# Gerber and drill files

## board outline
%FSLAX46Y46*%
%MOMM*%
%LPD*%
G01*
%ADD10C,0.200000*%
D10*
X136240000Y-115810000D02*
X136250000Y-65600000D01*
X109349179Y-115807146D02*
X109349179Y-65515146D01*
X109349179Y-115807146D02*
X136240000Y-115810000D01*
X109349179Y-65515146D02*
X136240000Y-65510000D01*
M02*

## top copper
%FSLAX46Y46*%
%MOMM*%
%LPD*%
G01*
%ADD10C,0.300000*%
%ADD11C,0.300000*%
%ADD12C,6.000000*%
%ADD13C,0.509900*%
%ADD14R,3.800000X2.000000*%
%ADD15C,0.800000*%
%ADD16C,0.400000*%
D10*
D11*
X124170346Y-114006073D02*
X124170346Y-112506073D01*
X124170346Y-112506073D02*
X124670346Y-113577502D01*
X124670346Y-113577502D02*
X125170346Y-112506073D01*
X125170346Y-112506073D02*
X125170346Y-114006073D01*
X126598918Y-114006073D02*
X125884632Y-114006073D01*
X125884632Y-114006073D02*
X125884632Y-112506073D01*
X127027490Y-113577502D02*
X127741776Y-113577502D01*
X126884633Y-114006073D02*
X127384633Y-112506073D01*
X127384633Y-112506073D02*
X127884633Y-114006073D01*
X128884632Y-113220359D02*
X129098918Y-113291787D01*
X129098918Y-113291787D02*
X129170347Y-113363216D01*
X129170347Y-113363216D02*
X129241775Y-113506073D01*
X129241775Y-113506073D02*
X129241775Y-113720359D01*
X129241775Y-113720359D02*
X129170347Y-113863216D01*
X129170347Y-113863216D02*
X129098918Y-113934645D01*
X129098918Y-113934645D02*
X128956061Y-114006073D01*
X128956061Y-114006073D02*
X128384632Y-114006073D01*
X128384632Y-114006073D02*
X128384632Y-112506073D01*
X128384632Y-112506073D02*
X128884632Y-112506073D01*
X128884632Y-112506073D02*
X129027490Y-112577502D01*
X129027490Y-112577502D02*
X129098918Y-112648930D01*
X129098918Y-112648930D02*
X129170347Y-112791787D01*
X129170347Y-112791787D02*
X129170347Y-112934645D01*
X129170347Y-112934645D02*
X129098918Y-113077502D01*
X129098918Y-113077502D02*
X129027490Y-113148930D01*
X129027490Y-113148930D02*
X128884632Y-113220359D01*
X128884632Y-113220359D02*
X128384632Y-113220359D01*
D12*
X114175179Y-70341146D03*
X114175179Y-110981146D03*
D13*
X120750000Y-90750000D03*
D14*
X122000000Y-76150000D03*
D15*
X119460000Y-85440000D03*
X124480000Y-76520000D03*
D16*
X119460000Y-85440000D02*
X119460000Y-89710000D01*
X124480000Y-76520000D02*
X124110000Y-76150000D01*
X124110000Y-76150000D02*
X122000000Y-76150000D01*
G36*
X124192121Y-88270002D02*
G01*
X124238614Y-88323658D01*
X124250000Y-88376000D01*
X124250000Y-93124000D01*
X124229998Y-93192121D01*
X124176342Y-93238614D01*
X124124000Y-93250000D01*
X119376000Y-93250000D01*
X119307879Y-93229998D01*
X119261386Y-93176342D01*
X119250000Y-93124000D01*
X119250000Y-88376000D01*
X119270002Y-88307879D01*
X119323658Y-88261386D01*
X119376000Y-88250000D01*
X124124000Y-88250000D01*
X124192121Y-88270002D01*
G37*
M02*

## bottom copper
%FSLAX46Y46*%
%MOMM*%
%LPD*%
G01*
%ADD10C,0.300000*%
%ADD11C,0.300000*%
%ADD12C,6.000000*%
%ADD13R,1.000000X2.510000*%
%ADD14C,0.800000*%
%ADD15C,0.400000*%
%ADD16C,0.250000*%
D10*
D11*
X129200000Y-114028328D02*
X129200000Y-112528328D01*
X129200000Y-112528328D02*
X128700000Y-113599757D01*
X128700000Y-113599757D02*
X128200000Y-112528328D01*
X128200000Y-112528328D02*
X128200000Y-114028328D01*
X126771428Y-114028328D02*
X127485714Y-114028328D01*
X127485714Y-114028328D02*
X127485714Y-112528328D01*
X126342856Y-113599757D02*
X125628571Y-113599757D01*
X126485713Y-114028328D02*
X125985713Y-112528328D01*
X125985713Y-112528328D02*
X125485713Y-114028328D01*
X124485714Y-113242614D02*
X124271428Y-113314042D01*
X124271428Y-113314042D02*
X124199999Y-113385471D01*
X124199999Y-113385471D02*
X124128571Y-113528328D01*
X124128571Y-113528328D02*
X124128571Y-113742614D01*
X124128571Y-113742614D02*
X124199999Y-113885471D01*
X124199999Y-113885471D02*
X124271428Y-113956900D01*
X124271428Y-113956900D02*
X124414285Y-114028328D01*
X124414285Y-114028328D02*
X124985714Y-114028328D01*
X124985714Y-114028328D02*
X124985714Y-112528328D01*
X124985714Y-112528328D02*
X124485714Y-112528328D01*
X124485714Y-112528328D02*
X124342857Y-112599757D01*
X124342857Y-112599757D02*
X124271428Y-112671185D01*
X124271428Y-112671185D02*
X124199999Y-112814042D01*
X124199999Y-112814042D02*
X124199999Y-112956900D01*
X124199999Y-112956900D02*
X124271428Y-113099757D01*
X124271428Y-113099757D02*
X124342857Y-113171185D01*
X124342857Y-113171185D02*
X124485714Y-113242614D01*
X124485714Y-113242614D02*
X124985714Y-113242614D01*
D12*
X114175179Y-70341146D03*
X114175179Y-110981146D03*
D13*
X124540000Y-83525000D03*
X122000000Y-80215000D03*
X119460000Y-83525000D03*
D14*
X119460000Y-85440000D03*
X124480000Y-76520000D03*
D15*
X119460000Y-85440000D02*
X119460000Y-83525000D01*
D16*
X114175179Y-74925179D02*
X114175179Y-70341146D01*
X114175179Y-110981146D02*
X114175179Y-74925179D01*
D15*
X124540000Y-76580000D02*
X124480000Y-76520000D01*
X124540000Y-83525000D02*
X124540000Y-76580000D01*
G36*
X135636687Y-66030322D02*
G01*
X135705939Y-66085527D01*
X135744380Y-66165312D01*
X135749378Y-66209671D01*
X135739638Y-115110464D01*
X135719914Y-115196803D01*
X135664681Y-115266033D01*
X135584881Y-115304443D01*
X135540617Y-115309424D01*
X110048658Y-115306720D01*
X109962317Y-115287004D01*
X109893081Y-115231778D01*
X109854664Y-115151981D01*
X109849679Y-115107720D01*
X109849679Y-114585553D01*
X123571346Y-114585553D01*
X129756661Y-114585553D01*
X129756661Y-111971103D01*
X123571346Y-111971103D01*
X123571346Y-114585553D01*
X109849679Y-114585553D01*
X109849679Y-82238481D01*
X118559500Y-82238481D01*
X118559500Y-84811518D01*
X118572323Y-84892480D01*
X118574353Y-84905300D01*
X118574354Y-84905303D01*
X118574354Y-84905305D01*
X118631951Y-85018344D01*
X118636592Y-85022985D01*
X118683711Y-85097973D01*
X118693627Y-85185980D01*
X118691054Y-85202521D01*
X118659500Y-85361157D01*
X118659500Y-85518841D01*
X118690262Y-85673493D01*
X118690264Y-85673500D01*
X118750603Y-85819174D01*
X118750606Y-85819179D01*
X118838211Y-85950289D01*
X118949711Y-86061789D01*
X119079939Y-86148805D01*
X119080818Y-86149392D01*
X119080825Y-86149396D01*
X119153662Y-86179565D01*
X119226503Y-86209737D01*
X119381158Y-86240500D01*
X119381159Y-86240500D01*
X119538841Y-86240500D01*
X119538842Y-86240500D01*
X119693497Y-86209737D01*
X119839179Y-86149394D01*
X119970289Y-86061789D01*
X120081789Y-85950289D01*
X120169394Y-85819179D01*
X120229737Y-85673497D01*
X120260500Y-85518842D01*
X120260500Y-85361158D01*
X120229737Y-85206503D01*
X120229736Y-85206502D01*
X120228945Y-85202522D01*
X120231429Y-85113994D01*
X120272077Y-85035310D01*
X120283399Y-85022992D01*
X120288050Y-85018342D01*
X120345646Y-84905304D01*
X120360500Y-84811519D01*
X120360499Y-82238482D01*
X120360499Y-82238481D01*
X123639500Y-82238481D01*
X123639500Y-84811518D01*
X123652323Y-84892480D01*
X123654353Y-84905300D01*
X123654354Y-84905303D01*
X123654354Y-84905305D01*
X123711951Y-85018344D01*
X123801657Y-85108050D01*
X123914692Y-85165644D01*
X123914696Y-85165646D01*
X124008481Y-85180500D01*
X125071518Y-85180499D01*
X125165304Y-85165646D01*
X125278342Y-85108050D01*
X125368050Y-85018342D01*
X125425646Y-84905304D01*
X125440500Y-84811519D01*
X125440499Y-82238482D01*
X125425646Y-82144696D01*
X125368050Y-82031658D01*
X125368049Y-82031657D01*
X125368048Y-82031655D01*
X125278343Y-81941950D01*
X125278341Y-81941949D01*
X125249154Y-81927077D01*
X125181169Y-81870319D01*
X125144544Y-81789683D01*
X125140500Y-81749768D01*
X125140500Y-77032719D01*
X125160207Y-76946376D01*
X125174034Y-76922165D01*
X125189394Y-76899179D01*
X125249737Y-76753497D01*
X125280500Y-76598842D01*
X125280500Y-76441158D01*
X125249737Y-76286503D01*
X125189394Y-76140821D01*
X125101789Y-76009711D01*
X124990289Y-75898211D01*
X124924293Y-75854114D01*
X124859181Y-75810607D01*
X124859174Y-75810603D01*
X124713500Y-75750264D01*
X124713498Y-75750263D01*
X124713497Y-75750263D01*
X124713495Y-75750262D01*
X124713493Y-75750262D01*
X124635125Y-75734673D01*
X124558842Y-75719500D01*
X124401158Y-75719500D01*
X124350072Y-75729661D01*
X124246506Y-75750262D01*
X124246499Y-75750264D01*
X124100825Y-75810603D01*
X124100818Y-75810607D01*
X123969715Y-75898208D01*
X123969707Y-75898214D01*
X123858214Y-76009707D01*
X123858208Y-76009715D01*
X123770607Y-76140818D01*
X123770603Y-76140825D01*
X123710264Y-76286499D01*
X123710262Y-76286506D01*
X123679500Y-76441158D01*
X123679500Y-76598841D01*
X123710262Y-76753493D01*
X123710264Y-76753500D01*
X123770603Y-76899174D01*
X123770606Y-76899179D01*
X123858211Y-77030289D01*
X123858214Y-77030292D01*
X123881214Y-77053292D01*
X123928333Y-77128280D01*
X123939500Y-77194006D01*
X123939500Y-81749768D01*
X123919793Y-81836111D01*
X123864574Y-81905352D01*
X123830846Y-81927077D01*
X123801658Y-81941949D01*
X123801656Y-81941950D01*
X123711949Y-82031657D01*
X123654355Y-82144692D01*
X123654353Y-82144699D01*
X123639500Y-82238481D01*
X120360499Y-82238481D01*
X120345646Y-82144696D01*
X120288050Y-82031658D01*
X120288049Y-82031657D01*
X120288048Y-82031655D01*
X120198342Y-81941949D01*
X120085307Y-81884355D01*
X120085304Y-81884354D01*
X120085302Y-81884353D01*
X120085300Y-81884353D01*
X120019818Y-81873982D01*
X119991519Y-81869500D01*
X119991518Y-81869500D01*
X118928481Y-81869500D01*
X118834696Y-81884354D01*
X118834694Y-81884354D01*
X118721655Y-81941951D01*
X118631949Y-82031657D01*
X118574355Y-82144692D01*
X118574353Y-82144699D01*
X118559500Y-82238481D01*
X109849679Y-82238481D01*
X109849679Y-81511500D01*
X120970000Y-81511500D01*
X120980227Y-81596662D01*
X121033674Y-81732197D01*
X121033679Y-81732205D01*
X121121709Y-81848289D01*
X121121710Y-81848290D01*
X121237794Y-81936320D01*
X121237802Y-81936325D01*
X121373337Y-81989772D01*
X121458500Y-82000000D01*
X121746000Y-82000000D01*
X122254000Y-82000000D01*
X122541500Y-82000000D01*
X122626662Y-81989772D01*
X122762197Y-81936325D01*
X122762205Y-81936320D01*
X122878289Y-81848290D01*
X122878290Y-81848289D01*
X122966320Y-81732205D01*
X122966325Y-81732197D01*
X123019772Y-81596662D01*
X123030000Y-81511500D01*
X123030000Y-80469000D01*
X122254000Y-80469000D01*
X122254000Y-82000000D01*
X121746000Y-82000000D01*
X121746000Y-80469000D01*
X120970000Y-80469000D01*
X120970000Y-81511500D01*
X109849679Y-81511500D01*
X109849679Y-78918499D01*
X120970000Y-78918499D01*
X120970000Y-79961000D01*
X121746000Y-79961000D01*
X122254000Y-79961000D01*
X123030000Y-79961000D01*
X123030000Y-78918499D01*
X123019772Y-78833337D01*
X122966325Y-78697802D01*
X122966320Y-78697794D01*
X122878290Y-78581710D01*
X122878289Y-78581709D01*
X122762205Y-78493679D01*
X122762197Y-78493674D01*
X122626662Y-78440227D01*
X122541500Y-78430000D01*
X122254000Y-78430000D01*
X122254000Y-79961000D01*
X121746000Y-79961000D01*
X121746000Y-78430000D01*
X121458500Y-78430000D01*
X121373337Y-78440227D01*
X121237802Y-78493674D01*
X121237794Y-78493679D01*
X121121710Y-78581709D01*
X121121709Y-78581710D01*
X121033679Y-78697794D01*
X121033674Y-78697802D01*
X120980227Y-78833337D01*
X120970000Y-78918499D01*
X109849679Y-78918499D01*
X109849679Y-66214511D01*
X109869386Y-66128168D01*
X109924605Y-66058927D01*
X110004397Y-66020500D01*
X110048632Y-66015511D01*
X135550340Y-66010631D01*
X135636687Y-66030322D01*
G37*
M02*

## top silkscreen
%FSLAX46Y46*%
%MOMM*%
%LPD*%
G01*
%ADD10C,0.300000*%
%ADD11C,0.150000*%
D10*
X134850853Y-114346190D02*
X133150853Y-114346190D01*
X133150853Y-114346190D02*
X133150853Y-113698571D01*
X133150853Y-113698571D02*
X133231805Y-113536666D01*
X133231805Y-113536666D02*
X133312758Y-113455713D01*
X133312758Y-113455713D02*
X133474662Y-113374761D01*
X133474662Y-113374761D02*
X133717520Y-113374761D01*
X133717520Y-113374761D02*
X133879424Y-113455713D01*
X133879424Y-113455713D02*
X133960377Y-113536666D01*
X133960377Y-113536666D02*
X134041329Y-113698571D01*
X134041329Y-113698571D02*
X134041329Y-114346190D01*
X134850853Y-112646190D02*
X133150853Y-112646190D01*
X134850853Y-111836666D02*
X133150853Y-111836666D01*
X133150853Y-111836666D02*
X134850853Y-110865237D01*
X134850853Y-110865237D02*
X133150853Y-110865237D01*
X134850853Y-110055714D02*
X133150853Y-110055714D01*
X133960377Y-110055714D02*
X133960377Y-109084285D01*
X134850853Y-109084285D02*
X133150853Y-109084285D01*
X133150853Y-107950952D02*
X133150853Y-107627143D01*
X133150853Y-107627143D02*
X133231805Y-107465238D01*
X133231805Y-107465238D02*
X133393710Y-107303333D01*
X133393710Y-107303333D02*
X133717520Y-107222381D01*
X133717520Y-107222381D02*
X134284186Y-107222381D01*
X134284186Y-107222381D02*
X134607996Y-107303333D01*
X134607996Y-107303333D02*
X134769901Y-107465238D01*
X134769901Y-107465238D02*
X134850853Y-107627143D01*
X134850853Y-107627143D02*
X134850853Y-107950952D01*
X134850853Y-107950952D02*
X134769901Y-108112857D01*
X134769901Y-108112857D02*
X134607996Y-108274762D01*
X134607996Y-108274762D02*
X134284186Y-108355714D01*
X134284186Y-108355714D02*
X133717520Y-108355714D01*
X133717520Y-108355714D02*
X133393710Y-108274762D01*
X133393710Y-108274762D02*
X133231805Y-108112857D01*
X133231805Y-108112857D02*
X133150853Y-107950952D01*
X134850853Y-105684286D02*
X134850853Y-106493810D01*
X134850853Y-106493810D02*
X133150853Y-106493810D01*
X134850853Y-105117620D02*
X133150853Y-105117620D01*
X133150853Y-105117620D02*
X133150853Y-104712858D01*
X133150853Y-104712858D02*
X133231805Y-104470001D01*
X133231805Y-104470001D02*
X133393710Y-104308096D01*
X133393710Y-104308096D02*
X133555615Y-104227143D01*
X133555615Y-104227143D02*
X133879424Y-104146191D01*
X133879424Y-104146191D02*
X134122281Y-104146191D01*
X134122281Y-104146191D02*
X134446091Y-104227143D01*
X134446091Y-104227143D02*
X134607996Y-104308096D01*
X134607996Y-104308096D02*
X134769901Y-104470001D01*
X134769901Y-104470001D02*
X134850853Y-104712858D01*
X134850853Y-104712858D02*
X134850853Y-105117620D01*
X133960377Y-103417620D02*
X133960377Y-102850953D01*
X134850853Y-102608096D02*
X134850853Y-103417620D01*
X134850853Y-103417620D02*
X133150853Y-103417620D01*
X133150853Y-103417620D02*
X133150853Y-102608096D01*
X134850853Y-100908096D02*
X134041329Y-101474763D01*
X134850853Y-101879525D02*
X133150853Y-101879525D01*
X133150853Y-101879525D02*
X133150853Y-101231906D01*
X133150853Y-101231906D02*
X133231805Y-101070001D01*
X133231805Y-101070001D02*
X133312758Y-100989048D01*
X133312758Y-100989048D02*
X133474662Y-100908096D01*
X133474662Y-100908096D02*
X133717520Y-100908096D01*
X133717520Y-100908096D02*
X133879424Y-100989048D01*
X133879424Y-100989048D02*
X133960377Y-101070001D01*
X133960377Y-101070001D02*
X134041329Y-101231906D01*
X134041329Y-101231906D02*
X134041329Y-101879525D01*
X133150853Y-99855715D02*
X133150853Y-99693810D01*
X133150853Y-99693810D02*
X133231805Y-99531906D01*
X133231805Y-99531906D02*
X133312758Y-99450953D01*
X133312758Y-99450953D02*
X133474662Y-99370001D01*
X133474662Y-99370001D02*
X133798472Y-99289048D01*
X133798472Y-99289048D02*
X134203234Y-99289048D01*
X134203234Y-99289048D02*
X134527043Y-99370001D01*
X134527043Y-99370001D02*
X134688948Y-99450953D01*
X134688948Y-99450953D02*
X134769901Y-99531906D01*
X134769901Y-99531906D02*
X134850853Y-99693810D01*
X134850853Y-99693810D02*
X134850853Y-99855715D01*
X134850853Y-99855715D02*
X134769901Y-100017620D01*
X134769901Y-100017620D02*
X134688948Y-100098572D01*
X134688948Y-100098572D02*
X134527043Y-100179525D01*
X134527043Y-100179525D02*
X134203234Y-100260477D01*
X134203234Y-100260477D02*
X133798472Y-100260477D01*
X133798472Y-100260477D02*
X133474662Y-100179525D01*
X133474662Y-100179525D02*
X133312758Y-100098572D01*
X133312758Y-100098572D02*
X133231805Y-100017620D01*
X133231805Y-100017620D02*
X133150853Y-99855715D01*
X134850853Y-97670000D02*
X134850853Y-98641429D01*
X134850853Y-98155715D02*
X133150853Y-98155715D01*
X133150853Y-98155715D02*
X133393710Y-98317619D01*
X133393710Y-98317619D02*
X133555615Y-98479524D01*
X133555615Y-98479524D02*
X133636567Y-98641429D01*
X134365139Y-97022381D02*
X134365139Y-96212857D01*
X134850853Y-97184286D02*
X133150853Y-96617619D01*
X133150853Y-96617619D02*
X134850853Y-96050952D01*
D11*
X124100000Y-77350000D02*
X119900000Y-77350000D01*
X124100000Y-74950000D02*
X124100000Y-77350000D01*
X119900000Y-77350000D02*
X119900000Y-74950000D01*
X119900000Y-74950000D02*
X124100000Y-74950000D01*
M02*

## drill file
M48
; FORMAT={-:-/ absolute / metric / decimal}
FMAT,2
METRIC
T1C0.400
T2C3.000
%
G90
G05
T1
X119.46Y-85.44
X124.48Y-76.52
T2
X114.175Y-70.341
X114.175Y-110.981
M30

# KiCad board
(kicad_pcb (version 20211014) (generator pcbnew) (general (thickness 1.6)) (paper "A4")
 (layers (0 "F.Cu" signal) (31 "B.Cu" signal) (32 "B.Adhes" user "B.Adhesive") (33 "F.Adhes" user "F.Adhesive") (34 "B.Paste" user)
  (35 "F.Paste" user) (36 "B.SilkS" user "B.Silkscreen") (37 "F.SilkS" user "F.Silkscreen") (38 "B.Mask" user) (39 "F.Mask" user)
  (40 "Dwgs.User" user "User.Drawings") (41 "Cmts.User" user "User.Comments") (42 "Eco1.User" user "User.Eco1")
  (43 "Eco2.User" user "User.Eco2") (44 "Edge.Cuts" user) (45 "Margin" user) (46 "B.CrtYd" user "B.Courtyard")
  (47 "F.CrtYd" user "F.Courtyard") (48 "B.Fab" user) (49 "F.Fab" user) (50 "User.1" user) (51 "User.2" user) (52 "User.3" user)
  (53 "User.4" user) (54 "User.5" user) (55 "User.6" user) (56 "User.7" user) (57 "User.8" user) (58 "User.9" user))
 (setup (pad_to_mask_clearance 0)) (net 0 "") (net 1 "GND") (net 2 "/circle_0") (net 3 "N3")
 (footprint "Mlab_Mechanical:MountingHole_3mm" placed (layer "F.Cu") (at 114.175179 70.341146)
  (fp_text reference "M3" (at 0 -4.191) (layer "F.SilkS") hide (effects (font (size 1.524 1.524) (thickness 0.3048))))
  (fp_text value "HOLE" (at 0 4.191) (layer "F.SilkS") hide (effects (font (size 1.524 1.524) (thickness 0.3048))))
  (pad "1" thru_hole circle locked (at 0 0) (size 6 6) (drill 3) (layers F&B.Cu *.Adhes *.Mask) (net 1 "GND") (clearance 1) (zone_connect 2)))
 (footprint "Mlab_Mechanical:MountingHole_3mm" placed (layer "F.Cu") (at 114.175179 110.981146)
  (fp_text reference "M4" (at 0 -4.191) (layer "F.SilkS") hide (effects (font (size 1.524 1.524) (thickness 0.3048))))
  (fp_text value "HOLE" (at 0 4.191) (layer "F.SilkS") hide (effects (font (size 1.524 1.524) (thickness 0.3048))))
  (pad "1" thru_hole circle locked (at 0 0) (size 6 6) (drill 3) (layers F&B.Cu *.Adhes *.Mask) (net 1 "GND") (clearance 1) (zone_connect 2)))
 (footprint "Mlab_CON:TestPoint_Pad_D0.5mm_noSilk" (layer "F.Cu") (at 120.75 90.75 90) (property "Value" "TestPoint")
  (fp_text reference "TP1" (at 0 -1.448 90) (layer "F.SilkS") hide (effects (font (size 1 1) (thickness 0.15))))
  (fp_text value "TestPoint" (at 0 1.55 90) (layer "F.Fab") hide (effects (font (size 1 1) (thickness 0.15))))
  (pad "1" smd circle (at 0 0 90) (size 0.5099 0.5099) (layers "F.Cu" "F.Mask") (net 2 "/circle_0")))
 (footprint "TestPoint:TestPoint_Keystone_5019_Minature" (layer "F.Cu") (at 122 76.15 180) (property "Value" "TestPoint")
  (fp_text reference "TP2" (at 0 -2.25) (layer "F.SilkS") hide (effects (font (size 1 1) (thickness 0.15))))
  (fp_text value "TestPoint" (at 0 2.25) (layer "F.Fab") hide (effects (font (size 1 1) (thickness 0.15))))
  (fp_line (start -2.1 -1.2) (end 2.1 -1.2) (layer "F.SilkS") (width 0.15))
  (fp_line (start -2.1 1.2) (end -2.1 -1.2) (layer "F.SilkS") (width 0.15))
  (fp_line (start 2.1 -1.2) (end 2.1 1.2) (layer "F.SilkS") (width 0.15))
  (fp_line (start 2.1 1.2) (end -2.1 1.2) (layer "F.SilkS") (width 0.15))
  (pad "1" smd rect (at 0 0 180) (size 3.8 2) (layers "F.Cu" "F.Paste" "F.Mask") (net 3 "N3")))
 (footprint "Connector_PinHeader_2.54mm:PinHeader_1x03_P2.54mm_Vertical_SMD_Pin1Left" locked (layer "B.Cu") (at 122 81.87 90)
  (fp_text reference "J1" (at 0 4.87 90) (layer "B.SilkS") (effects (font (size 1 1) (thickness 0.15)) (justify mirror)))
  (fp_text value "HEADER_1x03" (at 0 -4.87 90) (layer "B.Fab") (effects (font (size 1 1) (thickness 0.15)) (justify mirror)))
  (pad "1" smd rect locked (at -1.655 2.54 90) (size 2.51 1) (layers "B.Cu" "B.Paste" "B.Mask") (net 3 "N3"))
  (pad "2" smd rect locked (at 1.655 0 90) (size 2.51 1) (layers "B.Cu" "B.Paste" "B.Mask") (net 1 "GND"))
  (pad "3" smd rect locked (at -1.655 -2.54 90) (size 2.51 1) (layers "B.Cu" "B.Paste" "B.Mask") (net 2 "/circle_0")))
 (gr_line (start 136.24 115.81) (end 136.25 65.6) (layer "Edge.Cuts") (width 0.2))
 (gr_line (start 109.349179 115.807146) (end 109.349179 65.515146) (layer "Edge.Cuts") (width 0.2))
 (gr_line (start 109.349179 115.807146) (end 136.24 115.81) (layer "Edge.Cuts") (width 0.2))
 (gr_line (start 109.349179 65.515146) (end 136.24 65.51) (layer "Edge.Cuts") (width 0.2))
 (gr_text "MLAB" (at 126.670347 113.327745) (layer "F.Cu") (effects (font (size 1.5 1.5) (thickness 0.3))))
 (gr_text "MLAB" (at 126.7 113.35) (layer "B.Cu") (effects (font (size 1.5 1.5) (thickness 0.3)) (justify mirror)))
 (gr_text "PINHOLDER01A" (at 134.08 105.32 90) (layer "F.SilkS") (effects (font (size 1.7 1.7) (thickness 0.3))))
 (segment (start 119.46 85.44) (end 119.46 89.71) (width 0.4) (layer "F.Cu") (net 2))
 (via (at 119.46 85.44) (size 0.8) (drill 0.4) (layers "F.Cu" "B.Cu") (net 2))
 (segment (start 119.46 85.44) (end 119.46 83.525) (width 0.4) (layer "B.Cu") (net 2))
 (segment (start 114.175179 74.925179) (end 114.175179 70.341146) (width 0.25) (layer "B.Cu") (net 1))
 (segment (start 114.175179 110.981146) (end 114.175179 74.925179) (width 0.25) (layer "B.Cu") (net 1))
 (segment (start 124.48 76.52) (end 124.11 76.15) (width 0.4) (layer "F.Cu") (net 3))
 (segment (start 124.11 76.15) (end 122 76.15) (width 0.4) (layer "F.Cu") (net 3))
 (via (at 124.48 76.52) (size 0.8) (drill 0.4) (layers "F.Cu" "B.Cu") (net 3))
 (segment (start 124.54 76.58) (end 124.48 76.52) (width 0.4) (layer "B.Cu") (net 3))
 (segment (start 124.54 83.525) (end 124.54 76.58) (width 0.4) (layer "B.Cu") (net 3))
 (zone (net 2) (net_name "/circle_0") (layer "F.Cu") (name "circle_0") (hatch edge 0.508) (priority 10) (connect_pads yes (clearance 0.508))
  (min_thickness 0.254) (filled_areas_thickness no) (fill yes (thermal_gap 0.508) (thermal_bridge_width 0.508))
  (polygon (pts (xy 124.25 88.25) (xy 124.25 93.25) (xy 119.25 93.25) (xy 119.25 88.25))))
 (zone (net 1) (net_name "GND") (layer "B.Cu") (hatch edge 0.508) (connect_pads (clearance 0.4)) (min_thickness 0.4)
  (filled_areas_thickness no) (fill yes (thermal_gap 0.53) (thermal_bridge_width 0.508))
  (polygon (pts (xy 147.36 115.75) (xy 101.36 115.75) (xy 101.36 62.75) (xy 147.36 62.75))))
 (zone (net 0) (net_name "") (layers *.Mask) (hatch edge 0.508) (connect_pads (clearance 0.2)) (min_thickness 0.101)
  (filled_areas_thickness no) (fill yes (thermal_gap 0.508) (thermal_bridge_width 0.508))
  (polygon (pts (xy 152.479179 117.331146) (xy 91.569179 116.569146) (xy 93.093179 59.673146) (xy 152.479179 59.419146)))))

